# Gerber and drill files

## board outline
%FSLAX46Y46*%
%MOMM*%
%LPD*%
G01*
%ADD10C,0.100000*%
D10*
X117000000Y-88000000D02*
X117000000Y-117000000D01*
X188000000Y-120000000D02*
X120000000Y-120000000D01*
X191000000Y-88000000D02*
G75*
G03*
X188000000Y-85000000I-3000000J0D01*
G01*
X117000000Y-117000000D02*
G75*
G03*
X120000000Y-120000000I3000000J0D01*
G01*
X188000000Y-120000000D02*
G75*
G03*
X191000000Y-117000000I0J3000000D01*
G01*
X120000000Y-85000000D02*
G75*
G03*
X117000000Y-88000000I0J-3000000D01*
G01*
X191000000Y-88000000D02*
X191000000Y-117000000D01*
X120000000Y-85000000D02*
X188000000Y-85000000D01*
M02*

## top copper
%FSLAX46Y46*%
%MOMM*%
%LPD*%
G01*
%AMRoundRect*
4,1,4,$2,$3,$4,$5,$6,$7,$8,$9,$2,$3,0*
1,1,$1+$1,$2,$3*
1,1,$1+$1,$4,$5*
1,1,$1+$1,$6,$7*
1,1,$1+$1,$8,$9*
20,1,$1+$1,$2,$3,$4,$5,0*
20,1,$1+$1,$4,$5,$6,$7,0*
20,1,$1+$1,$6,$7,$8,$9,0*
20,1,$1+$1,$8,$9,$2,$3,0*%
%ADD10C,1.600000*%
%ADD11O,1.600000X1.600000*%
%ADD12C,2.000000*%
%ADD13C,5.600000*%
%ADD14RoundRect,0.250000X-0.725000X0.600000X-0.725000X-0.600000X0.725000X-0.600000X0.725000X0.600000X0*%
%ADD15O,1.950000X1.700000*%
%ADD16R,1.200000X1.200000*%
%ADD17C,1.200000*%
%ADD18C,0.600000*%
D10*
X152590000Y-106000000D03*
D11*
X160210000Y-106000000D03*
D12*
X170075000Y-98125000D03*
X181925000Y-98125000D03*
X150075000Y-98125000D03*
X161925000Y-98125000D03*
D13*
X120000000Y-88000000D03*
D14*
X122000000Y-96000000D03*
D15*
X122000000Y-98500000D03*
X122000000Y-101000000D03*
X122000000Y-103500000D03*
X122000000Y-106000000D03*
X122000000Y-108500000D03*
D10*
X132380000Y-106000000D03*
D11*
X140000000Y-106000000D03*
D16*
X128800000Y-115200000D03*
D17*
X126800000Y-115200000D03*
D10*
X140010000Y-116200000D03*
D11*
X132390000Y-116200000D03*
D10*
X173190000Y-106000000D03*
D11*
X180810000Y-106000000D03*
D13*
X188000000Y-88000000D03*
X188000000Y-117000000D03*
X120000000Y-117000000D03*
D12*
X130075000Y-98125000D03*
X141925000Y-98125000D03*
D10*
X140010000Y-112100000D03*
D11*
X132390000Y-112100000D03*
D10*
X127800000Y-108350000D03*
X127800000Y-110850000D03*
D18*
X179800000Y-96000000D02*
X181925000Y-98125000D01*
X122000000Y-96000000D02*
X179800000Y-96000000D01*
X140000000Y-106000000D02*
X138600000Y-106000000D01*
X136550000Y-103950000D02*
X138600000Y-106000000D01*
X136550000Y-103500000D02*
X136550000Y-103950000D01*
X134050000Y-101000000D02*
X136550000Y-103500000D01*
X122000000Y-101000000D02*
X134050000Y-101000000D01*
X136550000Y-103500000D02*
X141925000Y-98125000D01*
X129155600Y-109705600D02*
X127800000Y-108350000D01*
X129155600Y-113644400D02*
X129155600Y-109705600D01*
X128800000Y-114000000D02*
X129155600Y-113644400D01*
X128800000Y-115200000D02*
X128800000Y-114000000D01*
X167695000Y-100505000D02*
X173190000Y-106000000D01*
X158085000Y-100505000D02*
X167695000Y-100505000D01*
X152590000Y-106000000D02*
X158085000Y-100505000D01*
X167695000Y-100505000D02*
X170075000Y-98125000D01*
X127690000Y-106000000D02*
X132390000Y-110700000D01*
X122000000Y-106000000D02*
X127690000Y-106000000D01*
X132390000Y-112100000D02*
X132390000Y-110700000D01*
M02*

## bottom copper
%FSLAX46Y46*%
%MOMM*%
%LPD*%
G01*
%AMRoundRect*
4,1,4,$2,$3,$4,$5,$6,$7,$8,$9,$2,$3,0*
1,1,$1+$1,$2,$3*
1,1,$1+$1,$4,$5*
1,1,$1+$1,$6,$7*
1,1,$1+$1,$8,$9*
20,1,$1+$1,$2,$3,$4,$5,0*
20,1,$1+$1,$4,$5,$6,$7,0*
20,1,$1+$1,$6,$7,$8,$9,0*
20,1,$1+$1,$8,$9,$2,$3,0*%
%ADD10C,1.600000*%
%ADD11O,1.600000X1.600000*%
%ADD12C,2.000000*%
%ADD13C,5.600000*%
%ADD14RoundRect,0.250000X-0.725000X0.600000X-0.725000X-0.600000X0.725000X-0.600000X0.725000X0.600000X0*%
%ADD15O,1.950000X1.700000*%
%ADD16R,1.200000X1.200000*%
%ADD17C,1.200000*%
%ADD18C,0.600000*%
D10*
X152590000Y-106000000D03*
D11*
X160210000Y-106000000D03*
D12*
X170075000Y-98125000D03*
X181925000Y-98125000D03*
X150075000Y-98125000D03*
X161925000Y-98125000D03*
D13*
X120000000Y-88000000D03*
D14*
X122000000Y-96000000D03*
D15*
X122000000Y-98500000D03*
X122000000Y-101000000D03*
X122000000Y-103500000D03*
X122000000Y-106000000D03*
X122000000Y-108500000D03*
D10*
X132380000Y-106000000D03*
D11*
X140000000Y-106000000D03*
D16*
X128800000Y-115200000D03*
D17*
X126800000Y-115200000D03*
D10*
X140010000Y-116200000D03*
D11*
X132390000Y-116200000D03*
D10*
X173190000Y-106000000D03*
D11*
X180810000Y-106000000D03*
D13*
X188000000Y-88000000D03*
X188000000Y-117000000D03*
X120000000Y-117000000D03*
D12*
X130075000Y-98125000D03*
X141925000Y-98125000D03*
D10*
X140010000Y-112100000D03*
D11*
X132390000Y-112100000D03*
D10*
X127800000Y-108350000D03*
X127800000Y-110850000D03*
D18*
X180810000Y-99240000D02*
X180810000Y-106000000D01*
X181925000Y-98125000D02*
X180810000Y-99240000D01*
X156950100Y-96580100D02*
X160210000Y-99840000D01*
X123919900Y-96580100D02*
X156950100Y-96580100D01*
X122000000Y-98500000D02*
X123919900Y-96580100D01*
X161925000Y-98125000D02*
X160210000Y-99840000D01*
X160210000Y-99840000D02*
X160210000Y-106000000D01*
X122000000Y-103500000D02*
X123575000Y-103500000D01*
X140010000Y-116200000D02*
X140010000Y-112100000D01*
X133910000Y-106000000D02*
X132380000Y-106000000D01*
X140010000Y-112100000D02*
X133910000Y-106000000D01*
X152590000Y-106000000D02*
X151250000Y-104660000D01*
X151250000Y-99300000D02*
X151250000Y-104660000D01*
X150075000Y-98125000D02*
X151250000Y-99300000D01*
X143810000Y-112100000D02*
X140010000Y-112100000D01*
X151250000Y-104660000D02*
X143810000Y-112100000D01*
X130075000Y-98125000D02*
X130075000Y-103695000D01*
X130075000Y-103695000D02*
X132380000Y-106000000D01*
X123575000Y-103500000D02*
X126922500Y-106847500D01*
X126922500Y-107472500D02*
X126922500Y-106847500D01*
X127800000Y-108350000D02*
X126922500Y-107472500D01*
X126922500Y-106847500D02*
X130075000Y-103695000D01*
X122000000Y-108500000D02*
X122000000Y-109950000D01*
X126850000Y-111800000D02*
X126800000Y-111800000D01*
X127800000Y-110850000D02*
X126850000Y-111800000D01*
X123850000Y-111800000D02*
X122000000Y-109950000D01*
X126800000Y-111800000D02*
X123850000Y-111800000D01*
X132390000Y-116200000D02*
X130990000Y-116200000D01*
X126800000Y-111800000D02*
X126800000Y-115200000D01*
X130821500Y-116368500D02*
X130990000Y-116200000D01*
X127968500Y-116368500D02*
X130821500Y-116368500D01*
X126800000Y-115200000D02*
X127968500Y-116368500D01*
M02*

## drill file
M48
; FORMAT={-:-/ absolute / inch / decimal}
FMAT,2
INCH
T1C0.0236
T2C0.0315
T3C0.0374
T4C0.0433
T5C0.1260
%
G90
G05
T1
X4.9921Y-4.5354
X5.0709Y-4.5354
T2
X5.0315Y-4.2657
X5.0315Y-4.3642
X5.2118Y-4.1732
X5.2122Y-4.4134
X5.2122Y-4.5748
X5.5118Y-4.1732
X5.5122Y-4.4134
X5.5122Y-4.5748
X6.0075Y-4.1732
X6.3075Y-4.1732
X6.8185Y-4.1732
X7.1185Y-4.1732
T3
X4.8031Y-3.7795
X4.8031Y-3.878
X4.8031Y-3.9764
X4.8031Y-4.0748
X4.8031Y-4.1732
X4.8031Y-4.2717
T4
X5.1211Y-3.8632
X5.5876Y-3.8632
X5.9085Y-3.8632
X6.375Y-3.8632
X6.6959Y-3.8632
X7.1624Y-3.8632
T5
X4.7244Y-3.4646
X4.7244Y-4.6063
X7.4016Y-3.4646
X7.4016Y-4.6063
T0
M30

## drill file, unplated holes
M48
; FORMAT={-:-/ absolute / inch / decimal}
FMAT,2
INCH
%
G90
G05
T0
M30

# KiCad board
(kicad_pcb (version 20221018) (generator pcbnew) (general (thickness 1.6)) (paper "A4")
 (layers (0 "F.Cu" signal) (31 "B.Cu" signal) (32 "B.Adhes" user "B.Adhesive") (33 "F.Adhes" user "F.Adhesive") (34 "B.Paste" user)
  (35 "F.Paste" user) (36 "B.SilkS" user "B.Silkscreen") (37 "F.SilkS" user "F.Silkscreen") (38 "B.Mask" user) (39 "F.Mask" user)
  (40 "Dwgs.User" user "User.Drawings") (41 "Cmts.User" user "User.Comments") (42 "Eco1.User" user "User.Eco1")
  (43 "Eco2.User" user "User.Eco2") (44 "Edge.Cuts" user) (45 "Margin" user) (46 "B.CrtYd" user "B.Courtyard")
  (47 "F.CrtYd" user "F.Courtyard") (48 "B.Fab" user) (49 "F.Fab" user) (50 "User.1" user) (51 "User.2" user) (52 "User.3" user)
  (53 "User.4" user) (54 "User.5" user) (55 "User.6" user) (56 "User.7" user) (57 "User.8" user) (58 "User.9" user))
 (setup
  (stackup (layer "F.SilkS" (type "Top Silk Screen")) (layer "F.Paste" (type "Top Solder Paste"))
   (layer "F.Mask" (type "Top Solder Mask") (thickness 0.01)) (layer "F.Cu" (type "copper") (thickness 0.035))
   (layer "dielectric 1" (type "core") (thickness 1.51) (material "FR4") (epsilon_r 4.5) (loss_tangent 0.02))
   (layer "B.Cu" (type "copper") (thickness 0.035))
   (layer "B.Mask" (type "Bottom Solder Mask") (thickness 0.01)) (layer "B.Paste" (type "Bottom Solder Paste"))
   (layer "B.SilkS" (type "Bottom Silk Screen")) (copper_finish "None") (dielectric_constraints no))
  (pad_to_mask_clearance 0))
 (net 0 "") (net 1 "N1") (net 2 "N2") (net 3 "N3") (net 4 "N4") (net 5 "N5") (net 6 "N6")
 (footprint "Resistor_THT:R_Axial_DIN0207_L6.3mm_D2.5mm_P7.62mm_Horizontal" (layer "F.Cu") (at 152.59 106)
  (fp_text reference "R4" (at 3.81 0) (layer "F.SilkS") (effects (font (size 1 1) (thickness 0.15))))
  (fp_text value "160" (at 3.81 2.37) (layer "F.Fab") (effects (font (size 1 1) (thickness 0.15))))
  (pad "1" thru_hole circle (at 0 0) (size 1.6 1.6) (drill 0.8) (layers "*.Cu" "*.Mask") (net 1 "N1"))
  (pad "2" thru_hole oval (at 7.62 0) (size 1.6 1.6) (drill 0.8) (layers "*.Cu" "*.Mask") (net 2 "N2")))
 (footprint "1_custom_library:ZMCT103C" (layer "F.Cu") (at 167 93)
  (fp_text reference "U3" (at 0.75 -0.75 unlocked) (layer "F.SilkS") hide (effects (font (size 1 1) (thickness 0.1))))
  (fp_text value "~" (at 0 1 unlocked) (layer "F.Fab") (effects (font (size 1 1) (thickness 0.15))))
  (pad "1" thru_hole circle (at 3.075 5.125) (size 2 2) (drill 1.1) (layers "*.Cu" "*.Mask") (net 1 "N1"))
  (pad "2" thru_hole circle (at 14.925 5.125) (size 2 2) (drill 1.1) (layers "*.Cu" "*.Mask") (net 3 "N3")))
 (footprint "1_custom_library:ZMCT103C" (layer "F.Cu") (at 147 93)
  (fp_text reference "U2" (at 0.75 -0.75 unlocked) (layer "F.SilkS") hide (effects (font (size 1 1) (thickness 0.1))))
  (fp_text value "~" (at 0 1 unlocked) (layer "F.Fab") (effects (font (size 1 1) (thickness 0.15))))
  (pad "1" thru_hole circle (at 3.075 5.125) (size 2 2) (drill 1.1) (layers "*.Cu" "*.Mask") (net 1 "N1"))
  (pad "2" thru_hole circle (at 14.925 5.125) (size 2 2) (drill 1.1) (layers "*.Cu" "*.Mask") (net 2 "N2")))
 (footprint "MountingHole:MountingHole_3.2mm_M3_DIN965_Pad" (layer "F.Cu") (at 120 88)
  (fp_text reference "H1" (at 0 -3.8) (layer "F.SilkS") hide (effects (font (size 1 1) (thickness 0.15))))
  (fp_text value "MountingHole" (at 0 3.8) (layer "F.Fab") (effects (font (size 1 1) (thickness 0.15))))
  (pad "1" thru_hole circle (at 0 0) (size 5.6 5.6) (drill 3.2) (layers "*.Cu" "*.Mask")))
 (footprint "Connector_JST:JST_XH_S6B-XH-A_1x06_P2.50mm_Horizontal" (layer "F.Cu") (at 122 96 -90)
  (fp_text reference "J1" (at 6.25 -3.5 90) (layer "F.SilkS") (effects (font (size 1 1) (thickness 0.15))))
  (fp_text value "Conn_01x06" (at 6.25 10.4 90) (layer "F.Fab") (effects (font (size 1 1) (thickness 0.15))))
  (pad "1" thru_hole roundrect (at 0 0 270) (size 1.7 1.95) (drill 0.95) (layers "*.Cu" "*.Mask") (roundrect_rratio 0.1470588235)
   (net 3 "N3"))
  (pad "2" thru_hole oval (at 2.5 0 270) (size 1.7 1.95) (drill 0.95) (layers "*.Cu" "*.Mask") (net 2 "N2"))
  (pad "3" thru_hole oval (at 5 0 270) (size 1.7 1.95) (drill 0.95) (layers "*.Cu" "*.Mask") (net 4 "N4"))
  (pad "4" thru_hole oval (at 7.5 0 270) (size 1.7 1.95) (drill 0.95) (layers "*.Cu" "*.Mask") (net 1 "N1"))
  (pad "5" thru_hole oval (at 10 0 270) (size 1.7 1.95) (drill 0.95) (layers "*.Cu" "*.Mask") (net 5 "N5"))
  (pad "6" thru_hole oval (at 12.5 0 270) (size 1.7 1.95) (drill 0.95) (layers "*.Cu" "*.Mask") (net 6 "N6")))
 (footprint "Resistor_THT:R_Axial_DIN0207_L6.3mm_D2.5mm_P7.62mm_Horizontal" (layer "F.Cu") (at 132.38 106)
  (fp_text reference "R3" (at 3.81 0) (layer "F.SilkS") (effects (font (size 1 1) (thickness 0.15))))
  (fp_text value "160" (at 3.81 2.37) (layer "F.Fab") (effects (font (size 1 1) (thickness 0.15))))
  (pad "1" thru_hole circle (at 0 0) (size 1.6 1.6) (drill 0.8) (layers "*.Cu" "*.Mask") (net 1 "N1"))
  (pad "2" thru_hole oval (at 7.62 0) (size 1.6 1.6) (drill 0.8) (layers "*.Cu" "*.Mask") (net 4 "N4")))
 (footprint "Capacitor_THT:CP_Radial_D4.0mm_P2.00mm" (layer "F.Cu") (at 128.8 115.2 180)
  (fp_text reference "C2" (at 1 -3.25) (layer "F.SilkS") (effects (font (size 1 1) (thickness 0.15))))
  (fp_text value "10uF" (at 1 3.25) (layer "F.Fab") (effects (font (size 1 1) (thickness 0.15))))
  (pad "1" thru_hole rect (at 0 0 180) (size 1.2 1.2) (drill 0.6) (layers "*.Cu" "*.Mask") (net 1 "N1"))
  (pad "2" thru_hole circle (at 2 0 180) (size 1.2 1.2) (drill 0.6) (layers "*.Cu" "*.Mask") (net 6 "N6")))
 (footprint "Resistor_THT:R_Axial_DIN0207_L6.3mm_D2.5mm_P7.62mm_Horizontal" (layer "F.Cu") (at 140.01 116.2 180)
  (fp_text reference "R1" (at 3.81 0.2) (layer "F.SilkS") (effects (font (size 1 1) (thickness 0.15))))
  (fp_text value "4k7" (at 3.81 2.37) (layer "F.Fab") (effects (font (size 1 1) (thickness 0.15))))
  (pad "1" thru_hole circle (at 0 0 180) (size 1.6 1.6) (drill 0.8) (layers "*.Cu" "*.Mask") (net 1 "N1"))
  (pad "2" thru_hole oval (at 7.62 0 180) (size 1.6 1.6) (drill 0.8) (layers "*.Cu" "*.Mask") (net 6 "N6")))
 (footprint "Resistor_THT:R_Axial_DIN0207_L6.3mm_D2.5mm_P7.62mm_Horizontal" (layer "F.Cu") (at 173.19 106)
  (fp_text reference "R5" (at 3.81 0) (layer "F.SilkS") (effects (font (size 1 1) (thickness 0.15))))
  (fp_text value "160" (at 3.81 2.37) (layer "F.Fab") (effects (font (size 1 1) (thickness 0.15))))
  (pad "1" thru_hole circle (at 0 0) (size 1.6 1.6) (drill 0.8) (layers "*.Cu" "*.Mask") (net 1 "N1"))
  (pad "2" thru_hole oval (at 7.62 0) (size 1.6 1.6) (drill 0.8) (layers "*.Cu" "*.Mask") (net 3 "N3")))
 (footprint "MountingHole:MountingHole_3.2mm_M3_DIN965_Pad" (layer "F.Cu") (at 188 88)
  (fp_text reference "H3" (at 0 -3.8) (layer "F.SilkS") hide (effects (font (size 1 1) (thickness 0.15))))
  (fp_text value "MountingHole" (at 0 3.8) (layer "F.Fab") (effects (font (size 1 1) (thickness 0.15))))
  (pad "1" thru_hole circle (at 0 0) (size 5.6 5.6) (drill 3.2) (layers "*.Cu" "*.Mask")))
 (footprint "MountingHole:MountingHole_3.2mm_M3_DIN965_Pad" (layer "F.Cu") (at 188 117)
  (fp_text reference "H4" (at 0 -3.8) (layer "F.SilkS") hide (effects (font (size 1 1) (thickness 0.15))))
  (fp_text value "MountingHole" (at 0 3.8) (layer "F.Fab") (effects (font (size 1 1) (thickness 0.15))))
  (pad "1" thru_hole circle (at 0 0) (size 5.6 5.6) (drill 3.2) (layers "*.Cu" "*.Mask")))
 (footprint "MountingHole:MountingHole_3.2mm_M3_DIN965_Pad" (layer "F.Cu") (at 120 117)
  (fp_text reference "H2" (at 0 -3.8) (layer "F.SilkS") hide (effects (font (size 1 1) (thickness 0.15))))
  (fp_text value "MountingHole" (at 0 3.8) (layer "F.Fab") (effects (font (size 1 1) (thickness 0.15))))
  (pad "1" thru_hole circle (at 0 0) (size 5.6 5.6) (drill 3.2) (layers "*.Cu" "*.Mask")))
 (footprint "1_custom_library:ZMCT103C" (layer "F.Cu") (at 127 93)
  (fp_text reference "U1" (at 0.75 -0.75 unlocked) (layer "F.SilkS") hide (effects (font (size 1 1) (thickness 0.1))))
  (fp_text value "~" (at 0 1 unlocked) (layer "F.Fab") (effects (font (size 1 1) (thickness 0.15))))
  (pad "1" thru_hole circle (at 3.075 5.125) (size 2 2) (drill 1.1) (layers "*.Cu" "*.Mask") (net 1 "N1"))
  (pad "2" thru_hole circle (at 14.925 5.125) (size 2 2) (drill 1.1) (layers "*.Cu" "*.Mask") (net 4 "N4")))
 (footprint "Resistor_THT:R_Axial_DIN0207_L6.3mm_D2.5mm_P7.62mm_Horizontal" (layer "F.Cu") (at 140.01 112.1 180)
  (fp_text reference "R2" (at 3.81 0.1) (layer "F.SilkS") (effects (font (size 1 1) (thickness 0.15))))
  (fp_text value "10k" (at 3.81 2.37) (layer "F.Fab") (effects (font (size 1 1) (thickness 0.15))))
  (pad "1" thru_hole circle (at 0 0 180) (size 1.6 1.6) (drill 0.8) (layers "*.Cu" "*.Mask") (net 1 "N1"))
  (pad "2" thru_hole oval (at 7.62 0 180) (size 1.6 1.6) (drill 0.8) (layers "*.Cu" "*.Mask") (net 5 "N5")))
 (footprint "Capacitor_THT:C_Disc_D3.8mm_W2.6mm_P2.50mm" (layer "F.Cu") (at 127.8 108.35 -90)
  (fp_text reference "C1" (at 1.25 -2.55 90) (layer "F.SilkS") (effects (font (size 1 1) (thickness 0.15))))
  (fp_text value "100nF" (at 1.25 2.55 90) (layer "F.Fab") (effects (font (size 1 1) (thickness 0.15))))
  (pad "1" thru_hole circle (at 0 0 270) (size 1.6 1.6) (drill 0.8) (layers "*.Cu" "*.Mask") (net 1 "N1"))
  (pad "2" thru_hole circle (at 2.5 0 270) (size 1.6 1.6) (drill 0.8) (layers "*.Cu" "*.Mask") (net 6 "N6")))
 (gr_line (start 117 88) (end 117 117) (stroke (width 0.1) (type default)) (layer "Edge.Cuts"))
 (gr_line (start 188 120) (end 120 120) (stroke (width 0.1) (type default)) (layer "Edge.Cuts"))
 (gr_arc (start 188 85) (mid 190.12132 85.87868) (end 191 88) (stroke (width 0.1) (type default)) (layer "Edge.Cuts"))
 (gr_arc (start 120 120) (mid 117.87868 119.12132) (end 117 117) (stroke (width 0.1) (type default)) (layer "Edge.Cuts"))
 (gr_arc (start 191 117) (mid 190.12132 119.12132) (end 188 120) (stroke (width 0.1) (type default)) (layer "Edge.Cuts"))
 (gr_arc (start 117 88) (mid 117.87868 85.87868) (end 120 85) (stroke (width 0.1) (type default)) (layer "Edge.Cuts"))
 (gr_line (start 191 88) (end 191 117) (stroke (width 0.1) (type default)) (layer "Edge.Cuts"))
 (gr_line (start 120 85) (end 188 85) (stroke (width 0.1) (type default)) (layer "Edge.Cuts"))
 (segment (start 127.69 106) (end 132.39 110.7) (width 0.6) (layer "F.Cu") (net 5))
 (segment (start 132.39 112.1) (end 132.39 110.7) (width 0.6) (layer "F.Cu") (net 5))
 (segment (start 122 106) (end 127.69 106) (width 0.6) (layer "F.Cu") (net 5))
 (segment (start 132.39 116.2) (end 130.99 116.2) (width 0.6) (layer "B.Cu") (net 6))
 (segment (start 127.9685 116.3685) (end 130.8215 116.3685) (width 0.6) (layer "B.Cu") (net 6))
 (segment (start 126.8 111.8) (end 123.85 111.8) (width 0.6) (layer "B.Cu") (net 6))
 (segment (start 127.8 110.85) (end 126.85 111.8) (width 0.6) (layer "B.Cu") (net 6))
 (segment (start 130.8215 116.3685) (end 130.99 116.2) (width 0.6) (layer "B.Cu") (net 6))
 (segment (start 126.85 111.8) (end 126.8 111.8) (width 0.6) (layer "B.Cu") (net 6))
 (segment (start 126.8 115.2) (end 127.9685 116.3685) (width 0.6) (layer "B.Cu") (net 6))
 (segment (start 126.8 111.8) (end 126.8 115.2) (width 0.6) (layer "B.Cu") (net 6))
 (segment (start 122 108.5) (end 122 109.95) (width 0.6) (layer "B.Cu") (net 6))
 (segment (start 123.85 111.8) (end 122 109.95) (width 0.6) (layer "B.Cu") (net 6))
 (segment (start 167.695 100.505) (end 170.075 98.125) (width 0.6) (layer "F.Cu") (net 1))
 (segment (start 152.59 106) (end 158.085 100.505) (width 0.6) (layer "F.Cu") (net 1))
 (segment (start 158.085 100.505) (end 167.695 100.505) (width 0.6) (layer "F.Cu") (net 1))
 (segment (start 128.8 115.2) (end 128.8 114) (width 0.6) (layer "F.Cu") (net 1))
 (segment (start 167.695 100.505) (end 173.19 106) (width 0.6) (layer "F.Cu") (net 1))
 (segment (start 129.1556 113.6444) (end 129.1556 109.7056) (width 0.6) (layer "F.Cu") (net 1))
 (segment (start 129.1556 109.7056) (end 127.8 108.35) (width 0.6) (layer "F.Cu") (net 1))
 (segment (start 128.8 114) (end 129.1556 113.6444) (width 0.6) (layer "F.Cu") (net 1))
 (segment (start 140.01 116.2) (end 140.01 112.1) (width 0.6) (layer "B.Cu") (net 1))
 (segment (start 122 103.5) (end 123.575 103.5) (width 0.6) (layer "B.Cu") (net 1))
 (segment (start 126.9225 107.4725) (end 126.9225 106.8475) (width 0.6) (layer "B.Cu") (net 1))
 (segment (start 130.075 98.125) (end 130.075 103.695) (width 0.6) (layer "B.Cu") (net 1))
 (segment (start 140.01 112.1) (end 133.91 106) (width 0.6) (layer "B.Cu") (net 1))
 (segment (start 150.075 98.125) (end 151.25 99.3) (width 0.6) (layer "B.Cu") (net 1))
 (segment (start 130.075 103.695) (end 132.38 106) (width 0.6) (layer "B.Cu") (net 1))
 (segment (start 126.9225 106.8475) (end 130.075 103.695) (width 0.6) (layer "B.Cu") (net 1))
 (segment (start 133.91 106) (end 132.38 106) (width 0.6) (layer "B.Cu") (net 1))
 (segment (start 152.59 106) (end 151.25 104.66) (width 0.6) (layer "B.Cu") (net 1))
 (segment (start 151.25 99.3) (end 151.25 104.66) (width 0.6) (layer "B.Cu") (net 1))
 (segment (start 127.8 108.35) (end 126.9225 107.4725) (width 0.6) (layer "B.Cu") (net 1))
 (segment (start 143.81 112.1) (end 140.01 112.1) (width 0.6) (layer "B.Cu") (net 1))
 (segment (start 123.575 103.5) (end 126.9225 106.8475) (width 0.6) (layer "B.Cu") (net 1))
 (segment (start 151.25 104.66) (end 143.81 112.1) (width 0.6) (layer "B.Cu") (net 1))
 (segment (start 136.55 103.5) (end 136.55 103.95) (width 0.6) (layer "F.Cu") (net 4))
 (segment (start 140 106) (end 138.6 106) (width 0.6) (layer "F.Cu") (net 4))
 (segment (start 122 101) (end 134.05 101) (width 0.6) (layer "F.Cu") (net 4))
 (segment (start 134.05 101) (end 136.55 103.5) (width 0.6) (layer "F.Cu") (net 4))
 (segment (start 136.55 103.5) (end 141.925 98.125) (width 0.6) (layer "F.Cu") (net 4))
 (segment (start 136.55 103.95) (end 138.6 106) (width 0.6) (layer "F.Cu") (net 4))
 (segment (start 161.925 98.125) (end 160.21 99.84) (width 0.6) (layer "B.Cu") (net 2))
 (segment (start 156.9501 96.5801) (end 160.21 99.84) (width 0.6) (layer "B.Cu") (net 2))
 (segment (start 122 98.5) (end 123.9199 96.5801) (width 0.6) (layer "B.Cu") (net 2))
 (segment (start 160.21 99.84) (end 160.21 106) (width 0.6) (layer "B.Cu") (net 2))
 (segment (start 123.9199 96.5801) (end 156.9501 96.5801) (width 0.6) (layer "B.Cu") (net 2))
 (segment (start 122 96) (end 179.8 96) (width 0.6) (layer "F.Cu") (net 3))
 (segment (start 179.8 96) (end 181.925 98.125) (width 0.6) (layer "F.Cu") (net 3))
 (segment (start 180.81 99.24) (end 180.81 106) (width 0.6) (layer "B.Cu") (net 3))
 (segment (start 181.925 98.125) (end 180.81 99.24) (width 0.6) (layer "B.Cu") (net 3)))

